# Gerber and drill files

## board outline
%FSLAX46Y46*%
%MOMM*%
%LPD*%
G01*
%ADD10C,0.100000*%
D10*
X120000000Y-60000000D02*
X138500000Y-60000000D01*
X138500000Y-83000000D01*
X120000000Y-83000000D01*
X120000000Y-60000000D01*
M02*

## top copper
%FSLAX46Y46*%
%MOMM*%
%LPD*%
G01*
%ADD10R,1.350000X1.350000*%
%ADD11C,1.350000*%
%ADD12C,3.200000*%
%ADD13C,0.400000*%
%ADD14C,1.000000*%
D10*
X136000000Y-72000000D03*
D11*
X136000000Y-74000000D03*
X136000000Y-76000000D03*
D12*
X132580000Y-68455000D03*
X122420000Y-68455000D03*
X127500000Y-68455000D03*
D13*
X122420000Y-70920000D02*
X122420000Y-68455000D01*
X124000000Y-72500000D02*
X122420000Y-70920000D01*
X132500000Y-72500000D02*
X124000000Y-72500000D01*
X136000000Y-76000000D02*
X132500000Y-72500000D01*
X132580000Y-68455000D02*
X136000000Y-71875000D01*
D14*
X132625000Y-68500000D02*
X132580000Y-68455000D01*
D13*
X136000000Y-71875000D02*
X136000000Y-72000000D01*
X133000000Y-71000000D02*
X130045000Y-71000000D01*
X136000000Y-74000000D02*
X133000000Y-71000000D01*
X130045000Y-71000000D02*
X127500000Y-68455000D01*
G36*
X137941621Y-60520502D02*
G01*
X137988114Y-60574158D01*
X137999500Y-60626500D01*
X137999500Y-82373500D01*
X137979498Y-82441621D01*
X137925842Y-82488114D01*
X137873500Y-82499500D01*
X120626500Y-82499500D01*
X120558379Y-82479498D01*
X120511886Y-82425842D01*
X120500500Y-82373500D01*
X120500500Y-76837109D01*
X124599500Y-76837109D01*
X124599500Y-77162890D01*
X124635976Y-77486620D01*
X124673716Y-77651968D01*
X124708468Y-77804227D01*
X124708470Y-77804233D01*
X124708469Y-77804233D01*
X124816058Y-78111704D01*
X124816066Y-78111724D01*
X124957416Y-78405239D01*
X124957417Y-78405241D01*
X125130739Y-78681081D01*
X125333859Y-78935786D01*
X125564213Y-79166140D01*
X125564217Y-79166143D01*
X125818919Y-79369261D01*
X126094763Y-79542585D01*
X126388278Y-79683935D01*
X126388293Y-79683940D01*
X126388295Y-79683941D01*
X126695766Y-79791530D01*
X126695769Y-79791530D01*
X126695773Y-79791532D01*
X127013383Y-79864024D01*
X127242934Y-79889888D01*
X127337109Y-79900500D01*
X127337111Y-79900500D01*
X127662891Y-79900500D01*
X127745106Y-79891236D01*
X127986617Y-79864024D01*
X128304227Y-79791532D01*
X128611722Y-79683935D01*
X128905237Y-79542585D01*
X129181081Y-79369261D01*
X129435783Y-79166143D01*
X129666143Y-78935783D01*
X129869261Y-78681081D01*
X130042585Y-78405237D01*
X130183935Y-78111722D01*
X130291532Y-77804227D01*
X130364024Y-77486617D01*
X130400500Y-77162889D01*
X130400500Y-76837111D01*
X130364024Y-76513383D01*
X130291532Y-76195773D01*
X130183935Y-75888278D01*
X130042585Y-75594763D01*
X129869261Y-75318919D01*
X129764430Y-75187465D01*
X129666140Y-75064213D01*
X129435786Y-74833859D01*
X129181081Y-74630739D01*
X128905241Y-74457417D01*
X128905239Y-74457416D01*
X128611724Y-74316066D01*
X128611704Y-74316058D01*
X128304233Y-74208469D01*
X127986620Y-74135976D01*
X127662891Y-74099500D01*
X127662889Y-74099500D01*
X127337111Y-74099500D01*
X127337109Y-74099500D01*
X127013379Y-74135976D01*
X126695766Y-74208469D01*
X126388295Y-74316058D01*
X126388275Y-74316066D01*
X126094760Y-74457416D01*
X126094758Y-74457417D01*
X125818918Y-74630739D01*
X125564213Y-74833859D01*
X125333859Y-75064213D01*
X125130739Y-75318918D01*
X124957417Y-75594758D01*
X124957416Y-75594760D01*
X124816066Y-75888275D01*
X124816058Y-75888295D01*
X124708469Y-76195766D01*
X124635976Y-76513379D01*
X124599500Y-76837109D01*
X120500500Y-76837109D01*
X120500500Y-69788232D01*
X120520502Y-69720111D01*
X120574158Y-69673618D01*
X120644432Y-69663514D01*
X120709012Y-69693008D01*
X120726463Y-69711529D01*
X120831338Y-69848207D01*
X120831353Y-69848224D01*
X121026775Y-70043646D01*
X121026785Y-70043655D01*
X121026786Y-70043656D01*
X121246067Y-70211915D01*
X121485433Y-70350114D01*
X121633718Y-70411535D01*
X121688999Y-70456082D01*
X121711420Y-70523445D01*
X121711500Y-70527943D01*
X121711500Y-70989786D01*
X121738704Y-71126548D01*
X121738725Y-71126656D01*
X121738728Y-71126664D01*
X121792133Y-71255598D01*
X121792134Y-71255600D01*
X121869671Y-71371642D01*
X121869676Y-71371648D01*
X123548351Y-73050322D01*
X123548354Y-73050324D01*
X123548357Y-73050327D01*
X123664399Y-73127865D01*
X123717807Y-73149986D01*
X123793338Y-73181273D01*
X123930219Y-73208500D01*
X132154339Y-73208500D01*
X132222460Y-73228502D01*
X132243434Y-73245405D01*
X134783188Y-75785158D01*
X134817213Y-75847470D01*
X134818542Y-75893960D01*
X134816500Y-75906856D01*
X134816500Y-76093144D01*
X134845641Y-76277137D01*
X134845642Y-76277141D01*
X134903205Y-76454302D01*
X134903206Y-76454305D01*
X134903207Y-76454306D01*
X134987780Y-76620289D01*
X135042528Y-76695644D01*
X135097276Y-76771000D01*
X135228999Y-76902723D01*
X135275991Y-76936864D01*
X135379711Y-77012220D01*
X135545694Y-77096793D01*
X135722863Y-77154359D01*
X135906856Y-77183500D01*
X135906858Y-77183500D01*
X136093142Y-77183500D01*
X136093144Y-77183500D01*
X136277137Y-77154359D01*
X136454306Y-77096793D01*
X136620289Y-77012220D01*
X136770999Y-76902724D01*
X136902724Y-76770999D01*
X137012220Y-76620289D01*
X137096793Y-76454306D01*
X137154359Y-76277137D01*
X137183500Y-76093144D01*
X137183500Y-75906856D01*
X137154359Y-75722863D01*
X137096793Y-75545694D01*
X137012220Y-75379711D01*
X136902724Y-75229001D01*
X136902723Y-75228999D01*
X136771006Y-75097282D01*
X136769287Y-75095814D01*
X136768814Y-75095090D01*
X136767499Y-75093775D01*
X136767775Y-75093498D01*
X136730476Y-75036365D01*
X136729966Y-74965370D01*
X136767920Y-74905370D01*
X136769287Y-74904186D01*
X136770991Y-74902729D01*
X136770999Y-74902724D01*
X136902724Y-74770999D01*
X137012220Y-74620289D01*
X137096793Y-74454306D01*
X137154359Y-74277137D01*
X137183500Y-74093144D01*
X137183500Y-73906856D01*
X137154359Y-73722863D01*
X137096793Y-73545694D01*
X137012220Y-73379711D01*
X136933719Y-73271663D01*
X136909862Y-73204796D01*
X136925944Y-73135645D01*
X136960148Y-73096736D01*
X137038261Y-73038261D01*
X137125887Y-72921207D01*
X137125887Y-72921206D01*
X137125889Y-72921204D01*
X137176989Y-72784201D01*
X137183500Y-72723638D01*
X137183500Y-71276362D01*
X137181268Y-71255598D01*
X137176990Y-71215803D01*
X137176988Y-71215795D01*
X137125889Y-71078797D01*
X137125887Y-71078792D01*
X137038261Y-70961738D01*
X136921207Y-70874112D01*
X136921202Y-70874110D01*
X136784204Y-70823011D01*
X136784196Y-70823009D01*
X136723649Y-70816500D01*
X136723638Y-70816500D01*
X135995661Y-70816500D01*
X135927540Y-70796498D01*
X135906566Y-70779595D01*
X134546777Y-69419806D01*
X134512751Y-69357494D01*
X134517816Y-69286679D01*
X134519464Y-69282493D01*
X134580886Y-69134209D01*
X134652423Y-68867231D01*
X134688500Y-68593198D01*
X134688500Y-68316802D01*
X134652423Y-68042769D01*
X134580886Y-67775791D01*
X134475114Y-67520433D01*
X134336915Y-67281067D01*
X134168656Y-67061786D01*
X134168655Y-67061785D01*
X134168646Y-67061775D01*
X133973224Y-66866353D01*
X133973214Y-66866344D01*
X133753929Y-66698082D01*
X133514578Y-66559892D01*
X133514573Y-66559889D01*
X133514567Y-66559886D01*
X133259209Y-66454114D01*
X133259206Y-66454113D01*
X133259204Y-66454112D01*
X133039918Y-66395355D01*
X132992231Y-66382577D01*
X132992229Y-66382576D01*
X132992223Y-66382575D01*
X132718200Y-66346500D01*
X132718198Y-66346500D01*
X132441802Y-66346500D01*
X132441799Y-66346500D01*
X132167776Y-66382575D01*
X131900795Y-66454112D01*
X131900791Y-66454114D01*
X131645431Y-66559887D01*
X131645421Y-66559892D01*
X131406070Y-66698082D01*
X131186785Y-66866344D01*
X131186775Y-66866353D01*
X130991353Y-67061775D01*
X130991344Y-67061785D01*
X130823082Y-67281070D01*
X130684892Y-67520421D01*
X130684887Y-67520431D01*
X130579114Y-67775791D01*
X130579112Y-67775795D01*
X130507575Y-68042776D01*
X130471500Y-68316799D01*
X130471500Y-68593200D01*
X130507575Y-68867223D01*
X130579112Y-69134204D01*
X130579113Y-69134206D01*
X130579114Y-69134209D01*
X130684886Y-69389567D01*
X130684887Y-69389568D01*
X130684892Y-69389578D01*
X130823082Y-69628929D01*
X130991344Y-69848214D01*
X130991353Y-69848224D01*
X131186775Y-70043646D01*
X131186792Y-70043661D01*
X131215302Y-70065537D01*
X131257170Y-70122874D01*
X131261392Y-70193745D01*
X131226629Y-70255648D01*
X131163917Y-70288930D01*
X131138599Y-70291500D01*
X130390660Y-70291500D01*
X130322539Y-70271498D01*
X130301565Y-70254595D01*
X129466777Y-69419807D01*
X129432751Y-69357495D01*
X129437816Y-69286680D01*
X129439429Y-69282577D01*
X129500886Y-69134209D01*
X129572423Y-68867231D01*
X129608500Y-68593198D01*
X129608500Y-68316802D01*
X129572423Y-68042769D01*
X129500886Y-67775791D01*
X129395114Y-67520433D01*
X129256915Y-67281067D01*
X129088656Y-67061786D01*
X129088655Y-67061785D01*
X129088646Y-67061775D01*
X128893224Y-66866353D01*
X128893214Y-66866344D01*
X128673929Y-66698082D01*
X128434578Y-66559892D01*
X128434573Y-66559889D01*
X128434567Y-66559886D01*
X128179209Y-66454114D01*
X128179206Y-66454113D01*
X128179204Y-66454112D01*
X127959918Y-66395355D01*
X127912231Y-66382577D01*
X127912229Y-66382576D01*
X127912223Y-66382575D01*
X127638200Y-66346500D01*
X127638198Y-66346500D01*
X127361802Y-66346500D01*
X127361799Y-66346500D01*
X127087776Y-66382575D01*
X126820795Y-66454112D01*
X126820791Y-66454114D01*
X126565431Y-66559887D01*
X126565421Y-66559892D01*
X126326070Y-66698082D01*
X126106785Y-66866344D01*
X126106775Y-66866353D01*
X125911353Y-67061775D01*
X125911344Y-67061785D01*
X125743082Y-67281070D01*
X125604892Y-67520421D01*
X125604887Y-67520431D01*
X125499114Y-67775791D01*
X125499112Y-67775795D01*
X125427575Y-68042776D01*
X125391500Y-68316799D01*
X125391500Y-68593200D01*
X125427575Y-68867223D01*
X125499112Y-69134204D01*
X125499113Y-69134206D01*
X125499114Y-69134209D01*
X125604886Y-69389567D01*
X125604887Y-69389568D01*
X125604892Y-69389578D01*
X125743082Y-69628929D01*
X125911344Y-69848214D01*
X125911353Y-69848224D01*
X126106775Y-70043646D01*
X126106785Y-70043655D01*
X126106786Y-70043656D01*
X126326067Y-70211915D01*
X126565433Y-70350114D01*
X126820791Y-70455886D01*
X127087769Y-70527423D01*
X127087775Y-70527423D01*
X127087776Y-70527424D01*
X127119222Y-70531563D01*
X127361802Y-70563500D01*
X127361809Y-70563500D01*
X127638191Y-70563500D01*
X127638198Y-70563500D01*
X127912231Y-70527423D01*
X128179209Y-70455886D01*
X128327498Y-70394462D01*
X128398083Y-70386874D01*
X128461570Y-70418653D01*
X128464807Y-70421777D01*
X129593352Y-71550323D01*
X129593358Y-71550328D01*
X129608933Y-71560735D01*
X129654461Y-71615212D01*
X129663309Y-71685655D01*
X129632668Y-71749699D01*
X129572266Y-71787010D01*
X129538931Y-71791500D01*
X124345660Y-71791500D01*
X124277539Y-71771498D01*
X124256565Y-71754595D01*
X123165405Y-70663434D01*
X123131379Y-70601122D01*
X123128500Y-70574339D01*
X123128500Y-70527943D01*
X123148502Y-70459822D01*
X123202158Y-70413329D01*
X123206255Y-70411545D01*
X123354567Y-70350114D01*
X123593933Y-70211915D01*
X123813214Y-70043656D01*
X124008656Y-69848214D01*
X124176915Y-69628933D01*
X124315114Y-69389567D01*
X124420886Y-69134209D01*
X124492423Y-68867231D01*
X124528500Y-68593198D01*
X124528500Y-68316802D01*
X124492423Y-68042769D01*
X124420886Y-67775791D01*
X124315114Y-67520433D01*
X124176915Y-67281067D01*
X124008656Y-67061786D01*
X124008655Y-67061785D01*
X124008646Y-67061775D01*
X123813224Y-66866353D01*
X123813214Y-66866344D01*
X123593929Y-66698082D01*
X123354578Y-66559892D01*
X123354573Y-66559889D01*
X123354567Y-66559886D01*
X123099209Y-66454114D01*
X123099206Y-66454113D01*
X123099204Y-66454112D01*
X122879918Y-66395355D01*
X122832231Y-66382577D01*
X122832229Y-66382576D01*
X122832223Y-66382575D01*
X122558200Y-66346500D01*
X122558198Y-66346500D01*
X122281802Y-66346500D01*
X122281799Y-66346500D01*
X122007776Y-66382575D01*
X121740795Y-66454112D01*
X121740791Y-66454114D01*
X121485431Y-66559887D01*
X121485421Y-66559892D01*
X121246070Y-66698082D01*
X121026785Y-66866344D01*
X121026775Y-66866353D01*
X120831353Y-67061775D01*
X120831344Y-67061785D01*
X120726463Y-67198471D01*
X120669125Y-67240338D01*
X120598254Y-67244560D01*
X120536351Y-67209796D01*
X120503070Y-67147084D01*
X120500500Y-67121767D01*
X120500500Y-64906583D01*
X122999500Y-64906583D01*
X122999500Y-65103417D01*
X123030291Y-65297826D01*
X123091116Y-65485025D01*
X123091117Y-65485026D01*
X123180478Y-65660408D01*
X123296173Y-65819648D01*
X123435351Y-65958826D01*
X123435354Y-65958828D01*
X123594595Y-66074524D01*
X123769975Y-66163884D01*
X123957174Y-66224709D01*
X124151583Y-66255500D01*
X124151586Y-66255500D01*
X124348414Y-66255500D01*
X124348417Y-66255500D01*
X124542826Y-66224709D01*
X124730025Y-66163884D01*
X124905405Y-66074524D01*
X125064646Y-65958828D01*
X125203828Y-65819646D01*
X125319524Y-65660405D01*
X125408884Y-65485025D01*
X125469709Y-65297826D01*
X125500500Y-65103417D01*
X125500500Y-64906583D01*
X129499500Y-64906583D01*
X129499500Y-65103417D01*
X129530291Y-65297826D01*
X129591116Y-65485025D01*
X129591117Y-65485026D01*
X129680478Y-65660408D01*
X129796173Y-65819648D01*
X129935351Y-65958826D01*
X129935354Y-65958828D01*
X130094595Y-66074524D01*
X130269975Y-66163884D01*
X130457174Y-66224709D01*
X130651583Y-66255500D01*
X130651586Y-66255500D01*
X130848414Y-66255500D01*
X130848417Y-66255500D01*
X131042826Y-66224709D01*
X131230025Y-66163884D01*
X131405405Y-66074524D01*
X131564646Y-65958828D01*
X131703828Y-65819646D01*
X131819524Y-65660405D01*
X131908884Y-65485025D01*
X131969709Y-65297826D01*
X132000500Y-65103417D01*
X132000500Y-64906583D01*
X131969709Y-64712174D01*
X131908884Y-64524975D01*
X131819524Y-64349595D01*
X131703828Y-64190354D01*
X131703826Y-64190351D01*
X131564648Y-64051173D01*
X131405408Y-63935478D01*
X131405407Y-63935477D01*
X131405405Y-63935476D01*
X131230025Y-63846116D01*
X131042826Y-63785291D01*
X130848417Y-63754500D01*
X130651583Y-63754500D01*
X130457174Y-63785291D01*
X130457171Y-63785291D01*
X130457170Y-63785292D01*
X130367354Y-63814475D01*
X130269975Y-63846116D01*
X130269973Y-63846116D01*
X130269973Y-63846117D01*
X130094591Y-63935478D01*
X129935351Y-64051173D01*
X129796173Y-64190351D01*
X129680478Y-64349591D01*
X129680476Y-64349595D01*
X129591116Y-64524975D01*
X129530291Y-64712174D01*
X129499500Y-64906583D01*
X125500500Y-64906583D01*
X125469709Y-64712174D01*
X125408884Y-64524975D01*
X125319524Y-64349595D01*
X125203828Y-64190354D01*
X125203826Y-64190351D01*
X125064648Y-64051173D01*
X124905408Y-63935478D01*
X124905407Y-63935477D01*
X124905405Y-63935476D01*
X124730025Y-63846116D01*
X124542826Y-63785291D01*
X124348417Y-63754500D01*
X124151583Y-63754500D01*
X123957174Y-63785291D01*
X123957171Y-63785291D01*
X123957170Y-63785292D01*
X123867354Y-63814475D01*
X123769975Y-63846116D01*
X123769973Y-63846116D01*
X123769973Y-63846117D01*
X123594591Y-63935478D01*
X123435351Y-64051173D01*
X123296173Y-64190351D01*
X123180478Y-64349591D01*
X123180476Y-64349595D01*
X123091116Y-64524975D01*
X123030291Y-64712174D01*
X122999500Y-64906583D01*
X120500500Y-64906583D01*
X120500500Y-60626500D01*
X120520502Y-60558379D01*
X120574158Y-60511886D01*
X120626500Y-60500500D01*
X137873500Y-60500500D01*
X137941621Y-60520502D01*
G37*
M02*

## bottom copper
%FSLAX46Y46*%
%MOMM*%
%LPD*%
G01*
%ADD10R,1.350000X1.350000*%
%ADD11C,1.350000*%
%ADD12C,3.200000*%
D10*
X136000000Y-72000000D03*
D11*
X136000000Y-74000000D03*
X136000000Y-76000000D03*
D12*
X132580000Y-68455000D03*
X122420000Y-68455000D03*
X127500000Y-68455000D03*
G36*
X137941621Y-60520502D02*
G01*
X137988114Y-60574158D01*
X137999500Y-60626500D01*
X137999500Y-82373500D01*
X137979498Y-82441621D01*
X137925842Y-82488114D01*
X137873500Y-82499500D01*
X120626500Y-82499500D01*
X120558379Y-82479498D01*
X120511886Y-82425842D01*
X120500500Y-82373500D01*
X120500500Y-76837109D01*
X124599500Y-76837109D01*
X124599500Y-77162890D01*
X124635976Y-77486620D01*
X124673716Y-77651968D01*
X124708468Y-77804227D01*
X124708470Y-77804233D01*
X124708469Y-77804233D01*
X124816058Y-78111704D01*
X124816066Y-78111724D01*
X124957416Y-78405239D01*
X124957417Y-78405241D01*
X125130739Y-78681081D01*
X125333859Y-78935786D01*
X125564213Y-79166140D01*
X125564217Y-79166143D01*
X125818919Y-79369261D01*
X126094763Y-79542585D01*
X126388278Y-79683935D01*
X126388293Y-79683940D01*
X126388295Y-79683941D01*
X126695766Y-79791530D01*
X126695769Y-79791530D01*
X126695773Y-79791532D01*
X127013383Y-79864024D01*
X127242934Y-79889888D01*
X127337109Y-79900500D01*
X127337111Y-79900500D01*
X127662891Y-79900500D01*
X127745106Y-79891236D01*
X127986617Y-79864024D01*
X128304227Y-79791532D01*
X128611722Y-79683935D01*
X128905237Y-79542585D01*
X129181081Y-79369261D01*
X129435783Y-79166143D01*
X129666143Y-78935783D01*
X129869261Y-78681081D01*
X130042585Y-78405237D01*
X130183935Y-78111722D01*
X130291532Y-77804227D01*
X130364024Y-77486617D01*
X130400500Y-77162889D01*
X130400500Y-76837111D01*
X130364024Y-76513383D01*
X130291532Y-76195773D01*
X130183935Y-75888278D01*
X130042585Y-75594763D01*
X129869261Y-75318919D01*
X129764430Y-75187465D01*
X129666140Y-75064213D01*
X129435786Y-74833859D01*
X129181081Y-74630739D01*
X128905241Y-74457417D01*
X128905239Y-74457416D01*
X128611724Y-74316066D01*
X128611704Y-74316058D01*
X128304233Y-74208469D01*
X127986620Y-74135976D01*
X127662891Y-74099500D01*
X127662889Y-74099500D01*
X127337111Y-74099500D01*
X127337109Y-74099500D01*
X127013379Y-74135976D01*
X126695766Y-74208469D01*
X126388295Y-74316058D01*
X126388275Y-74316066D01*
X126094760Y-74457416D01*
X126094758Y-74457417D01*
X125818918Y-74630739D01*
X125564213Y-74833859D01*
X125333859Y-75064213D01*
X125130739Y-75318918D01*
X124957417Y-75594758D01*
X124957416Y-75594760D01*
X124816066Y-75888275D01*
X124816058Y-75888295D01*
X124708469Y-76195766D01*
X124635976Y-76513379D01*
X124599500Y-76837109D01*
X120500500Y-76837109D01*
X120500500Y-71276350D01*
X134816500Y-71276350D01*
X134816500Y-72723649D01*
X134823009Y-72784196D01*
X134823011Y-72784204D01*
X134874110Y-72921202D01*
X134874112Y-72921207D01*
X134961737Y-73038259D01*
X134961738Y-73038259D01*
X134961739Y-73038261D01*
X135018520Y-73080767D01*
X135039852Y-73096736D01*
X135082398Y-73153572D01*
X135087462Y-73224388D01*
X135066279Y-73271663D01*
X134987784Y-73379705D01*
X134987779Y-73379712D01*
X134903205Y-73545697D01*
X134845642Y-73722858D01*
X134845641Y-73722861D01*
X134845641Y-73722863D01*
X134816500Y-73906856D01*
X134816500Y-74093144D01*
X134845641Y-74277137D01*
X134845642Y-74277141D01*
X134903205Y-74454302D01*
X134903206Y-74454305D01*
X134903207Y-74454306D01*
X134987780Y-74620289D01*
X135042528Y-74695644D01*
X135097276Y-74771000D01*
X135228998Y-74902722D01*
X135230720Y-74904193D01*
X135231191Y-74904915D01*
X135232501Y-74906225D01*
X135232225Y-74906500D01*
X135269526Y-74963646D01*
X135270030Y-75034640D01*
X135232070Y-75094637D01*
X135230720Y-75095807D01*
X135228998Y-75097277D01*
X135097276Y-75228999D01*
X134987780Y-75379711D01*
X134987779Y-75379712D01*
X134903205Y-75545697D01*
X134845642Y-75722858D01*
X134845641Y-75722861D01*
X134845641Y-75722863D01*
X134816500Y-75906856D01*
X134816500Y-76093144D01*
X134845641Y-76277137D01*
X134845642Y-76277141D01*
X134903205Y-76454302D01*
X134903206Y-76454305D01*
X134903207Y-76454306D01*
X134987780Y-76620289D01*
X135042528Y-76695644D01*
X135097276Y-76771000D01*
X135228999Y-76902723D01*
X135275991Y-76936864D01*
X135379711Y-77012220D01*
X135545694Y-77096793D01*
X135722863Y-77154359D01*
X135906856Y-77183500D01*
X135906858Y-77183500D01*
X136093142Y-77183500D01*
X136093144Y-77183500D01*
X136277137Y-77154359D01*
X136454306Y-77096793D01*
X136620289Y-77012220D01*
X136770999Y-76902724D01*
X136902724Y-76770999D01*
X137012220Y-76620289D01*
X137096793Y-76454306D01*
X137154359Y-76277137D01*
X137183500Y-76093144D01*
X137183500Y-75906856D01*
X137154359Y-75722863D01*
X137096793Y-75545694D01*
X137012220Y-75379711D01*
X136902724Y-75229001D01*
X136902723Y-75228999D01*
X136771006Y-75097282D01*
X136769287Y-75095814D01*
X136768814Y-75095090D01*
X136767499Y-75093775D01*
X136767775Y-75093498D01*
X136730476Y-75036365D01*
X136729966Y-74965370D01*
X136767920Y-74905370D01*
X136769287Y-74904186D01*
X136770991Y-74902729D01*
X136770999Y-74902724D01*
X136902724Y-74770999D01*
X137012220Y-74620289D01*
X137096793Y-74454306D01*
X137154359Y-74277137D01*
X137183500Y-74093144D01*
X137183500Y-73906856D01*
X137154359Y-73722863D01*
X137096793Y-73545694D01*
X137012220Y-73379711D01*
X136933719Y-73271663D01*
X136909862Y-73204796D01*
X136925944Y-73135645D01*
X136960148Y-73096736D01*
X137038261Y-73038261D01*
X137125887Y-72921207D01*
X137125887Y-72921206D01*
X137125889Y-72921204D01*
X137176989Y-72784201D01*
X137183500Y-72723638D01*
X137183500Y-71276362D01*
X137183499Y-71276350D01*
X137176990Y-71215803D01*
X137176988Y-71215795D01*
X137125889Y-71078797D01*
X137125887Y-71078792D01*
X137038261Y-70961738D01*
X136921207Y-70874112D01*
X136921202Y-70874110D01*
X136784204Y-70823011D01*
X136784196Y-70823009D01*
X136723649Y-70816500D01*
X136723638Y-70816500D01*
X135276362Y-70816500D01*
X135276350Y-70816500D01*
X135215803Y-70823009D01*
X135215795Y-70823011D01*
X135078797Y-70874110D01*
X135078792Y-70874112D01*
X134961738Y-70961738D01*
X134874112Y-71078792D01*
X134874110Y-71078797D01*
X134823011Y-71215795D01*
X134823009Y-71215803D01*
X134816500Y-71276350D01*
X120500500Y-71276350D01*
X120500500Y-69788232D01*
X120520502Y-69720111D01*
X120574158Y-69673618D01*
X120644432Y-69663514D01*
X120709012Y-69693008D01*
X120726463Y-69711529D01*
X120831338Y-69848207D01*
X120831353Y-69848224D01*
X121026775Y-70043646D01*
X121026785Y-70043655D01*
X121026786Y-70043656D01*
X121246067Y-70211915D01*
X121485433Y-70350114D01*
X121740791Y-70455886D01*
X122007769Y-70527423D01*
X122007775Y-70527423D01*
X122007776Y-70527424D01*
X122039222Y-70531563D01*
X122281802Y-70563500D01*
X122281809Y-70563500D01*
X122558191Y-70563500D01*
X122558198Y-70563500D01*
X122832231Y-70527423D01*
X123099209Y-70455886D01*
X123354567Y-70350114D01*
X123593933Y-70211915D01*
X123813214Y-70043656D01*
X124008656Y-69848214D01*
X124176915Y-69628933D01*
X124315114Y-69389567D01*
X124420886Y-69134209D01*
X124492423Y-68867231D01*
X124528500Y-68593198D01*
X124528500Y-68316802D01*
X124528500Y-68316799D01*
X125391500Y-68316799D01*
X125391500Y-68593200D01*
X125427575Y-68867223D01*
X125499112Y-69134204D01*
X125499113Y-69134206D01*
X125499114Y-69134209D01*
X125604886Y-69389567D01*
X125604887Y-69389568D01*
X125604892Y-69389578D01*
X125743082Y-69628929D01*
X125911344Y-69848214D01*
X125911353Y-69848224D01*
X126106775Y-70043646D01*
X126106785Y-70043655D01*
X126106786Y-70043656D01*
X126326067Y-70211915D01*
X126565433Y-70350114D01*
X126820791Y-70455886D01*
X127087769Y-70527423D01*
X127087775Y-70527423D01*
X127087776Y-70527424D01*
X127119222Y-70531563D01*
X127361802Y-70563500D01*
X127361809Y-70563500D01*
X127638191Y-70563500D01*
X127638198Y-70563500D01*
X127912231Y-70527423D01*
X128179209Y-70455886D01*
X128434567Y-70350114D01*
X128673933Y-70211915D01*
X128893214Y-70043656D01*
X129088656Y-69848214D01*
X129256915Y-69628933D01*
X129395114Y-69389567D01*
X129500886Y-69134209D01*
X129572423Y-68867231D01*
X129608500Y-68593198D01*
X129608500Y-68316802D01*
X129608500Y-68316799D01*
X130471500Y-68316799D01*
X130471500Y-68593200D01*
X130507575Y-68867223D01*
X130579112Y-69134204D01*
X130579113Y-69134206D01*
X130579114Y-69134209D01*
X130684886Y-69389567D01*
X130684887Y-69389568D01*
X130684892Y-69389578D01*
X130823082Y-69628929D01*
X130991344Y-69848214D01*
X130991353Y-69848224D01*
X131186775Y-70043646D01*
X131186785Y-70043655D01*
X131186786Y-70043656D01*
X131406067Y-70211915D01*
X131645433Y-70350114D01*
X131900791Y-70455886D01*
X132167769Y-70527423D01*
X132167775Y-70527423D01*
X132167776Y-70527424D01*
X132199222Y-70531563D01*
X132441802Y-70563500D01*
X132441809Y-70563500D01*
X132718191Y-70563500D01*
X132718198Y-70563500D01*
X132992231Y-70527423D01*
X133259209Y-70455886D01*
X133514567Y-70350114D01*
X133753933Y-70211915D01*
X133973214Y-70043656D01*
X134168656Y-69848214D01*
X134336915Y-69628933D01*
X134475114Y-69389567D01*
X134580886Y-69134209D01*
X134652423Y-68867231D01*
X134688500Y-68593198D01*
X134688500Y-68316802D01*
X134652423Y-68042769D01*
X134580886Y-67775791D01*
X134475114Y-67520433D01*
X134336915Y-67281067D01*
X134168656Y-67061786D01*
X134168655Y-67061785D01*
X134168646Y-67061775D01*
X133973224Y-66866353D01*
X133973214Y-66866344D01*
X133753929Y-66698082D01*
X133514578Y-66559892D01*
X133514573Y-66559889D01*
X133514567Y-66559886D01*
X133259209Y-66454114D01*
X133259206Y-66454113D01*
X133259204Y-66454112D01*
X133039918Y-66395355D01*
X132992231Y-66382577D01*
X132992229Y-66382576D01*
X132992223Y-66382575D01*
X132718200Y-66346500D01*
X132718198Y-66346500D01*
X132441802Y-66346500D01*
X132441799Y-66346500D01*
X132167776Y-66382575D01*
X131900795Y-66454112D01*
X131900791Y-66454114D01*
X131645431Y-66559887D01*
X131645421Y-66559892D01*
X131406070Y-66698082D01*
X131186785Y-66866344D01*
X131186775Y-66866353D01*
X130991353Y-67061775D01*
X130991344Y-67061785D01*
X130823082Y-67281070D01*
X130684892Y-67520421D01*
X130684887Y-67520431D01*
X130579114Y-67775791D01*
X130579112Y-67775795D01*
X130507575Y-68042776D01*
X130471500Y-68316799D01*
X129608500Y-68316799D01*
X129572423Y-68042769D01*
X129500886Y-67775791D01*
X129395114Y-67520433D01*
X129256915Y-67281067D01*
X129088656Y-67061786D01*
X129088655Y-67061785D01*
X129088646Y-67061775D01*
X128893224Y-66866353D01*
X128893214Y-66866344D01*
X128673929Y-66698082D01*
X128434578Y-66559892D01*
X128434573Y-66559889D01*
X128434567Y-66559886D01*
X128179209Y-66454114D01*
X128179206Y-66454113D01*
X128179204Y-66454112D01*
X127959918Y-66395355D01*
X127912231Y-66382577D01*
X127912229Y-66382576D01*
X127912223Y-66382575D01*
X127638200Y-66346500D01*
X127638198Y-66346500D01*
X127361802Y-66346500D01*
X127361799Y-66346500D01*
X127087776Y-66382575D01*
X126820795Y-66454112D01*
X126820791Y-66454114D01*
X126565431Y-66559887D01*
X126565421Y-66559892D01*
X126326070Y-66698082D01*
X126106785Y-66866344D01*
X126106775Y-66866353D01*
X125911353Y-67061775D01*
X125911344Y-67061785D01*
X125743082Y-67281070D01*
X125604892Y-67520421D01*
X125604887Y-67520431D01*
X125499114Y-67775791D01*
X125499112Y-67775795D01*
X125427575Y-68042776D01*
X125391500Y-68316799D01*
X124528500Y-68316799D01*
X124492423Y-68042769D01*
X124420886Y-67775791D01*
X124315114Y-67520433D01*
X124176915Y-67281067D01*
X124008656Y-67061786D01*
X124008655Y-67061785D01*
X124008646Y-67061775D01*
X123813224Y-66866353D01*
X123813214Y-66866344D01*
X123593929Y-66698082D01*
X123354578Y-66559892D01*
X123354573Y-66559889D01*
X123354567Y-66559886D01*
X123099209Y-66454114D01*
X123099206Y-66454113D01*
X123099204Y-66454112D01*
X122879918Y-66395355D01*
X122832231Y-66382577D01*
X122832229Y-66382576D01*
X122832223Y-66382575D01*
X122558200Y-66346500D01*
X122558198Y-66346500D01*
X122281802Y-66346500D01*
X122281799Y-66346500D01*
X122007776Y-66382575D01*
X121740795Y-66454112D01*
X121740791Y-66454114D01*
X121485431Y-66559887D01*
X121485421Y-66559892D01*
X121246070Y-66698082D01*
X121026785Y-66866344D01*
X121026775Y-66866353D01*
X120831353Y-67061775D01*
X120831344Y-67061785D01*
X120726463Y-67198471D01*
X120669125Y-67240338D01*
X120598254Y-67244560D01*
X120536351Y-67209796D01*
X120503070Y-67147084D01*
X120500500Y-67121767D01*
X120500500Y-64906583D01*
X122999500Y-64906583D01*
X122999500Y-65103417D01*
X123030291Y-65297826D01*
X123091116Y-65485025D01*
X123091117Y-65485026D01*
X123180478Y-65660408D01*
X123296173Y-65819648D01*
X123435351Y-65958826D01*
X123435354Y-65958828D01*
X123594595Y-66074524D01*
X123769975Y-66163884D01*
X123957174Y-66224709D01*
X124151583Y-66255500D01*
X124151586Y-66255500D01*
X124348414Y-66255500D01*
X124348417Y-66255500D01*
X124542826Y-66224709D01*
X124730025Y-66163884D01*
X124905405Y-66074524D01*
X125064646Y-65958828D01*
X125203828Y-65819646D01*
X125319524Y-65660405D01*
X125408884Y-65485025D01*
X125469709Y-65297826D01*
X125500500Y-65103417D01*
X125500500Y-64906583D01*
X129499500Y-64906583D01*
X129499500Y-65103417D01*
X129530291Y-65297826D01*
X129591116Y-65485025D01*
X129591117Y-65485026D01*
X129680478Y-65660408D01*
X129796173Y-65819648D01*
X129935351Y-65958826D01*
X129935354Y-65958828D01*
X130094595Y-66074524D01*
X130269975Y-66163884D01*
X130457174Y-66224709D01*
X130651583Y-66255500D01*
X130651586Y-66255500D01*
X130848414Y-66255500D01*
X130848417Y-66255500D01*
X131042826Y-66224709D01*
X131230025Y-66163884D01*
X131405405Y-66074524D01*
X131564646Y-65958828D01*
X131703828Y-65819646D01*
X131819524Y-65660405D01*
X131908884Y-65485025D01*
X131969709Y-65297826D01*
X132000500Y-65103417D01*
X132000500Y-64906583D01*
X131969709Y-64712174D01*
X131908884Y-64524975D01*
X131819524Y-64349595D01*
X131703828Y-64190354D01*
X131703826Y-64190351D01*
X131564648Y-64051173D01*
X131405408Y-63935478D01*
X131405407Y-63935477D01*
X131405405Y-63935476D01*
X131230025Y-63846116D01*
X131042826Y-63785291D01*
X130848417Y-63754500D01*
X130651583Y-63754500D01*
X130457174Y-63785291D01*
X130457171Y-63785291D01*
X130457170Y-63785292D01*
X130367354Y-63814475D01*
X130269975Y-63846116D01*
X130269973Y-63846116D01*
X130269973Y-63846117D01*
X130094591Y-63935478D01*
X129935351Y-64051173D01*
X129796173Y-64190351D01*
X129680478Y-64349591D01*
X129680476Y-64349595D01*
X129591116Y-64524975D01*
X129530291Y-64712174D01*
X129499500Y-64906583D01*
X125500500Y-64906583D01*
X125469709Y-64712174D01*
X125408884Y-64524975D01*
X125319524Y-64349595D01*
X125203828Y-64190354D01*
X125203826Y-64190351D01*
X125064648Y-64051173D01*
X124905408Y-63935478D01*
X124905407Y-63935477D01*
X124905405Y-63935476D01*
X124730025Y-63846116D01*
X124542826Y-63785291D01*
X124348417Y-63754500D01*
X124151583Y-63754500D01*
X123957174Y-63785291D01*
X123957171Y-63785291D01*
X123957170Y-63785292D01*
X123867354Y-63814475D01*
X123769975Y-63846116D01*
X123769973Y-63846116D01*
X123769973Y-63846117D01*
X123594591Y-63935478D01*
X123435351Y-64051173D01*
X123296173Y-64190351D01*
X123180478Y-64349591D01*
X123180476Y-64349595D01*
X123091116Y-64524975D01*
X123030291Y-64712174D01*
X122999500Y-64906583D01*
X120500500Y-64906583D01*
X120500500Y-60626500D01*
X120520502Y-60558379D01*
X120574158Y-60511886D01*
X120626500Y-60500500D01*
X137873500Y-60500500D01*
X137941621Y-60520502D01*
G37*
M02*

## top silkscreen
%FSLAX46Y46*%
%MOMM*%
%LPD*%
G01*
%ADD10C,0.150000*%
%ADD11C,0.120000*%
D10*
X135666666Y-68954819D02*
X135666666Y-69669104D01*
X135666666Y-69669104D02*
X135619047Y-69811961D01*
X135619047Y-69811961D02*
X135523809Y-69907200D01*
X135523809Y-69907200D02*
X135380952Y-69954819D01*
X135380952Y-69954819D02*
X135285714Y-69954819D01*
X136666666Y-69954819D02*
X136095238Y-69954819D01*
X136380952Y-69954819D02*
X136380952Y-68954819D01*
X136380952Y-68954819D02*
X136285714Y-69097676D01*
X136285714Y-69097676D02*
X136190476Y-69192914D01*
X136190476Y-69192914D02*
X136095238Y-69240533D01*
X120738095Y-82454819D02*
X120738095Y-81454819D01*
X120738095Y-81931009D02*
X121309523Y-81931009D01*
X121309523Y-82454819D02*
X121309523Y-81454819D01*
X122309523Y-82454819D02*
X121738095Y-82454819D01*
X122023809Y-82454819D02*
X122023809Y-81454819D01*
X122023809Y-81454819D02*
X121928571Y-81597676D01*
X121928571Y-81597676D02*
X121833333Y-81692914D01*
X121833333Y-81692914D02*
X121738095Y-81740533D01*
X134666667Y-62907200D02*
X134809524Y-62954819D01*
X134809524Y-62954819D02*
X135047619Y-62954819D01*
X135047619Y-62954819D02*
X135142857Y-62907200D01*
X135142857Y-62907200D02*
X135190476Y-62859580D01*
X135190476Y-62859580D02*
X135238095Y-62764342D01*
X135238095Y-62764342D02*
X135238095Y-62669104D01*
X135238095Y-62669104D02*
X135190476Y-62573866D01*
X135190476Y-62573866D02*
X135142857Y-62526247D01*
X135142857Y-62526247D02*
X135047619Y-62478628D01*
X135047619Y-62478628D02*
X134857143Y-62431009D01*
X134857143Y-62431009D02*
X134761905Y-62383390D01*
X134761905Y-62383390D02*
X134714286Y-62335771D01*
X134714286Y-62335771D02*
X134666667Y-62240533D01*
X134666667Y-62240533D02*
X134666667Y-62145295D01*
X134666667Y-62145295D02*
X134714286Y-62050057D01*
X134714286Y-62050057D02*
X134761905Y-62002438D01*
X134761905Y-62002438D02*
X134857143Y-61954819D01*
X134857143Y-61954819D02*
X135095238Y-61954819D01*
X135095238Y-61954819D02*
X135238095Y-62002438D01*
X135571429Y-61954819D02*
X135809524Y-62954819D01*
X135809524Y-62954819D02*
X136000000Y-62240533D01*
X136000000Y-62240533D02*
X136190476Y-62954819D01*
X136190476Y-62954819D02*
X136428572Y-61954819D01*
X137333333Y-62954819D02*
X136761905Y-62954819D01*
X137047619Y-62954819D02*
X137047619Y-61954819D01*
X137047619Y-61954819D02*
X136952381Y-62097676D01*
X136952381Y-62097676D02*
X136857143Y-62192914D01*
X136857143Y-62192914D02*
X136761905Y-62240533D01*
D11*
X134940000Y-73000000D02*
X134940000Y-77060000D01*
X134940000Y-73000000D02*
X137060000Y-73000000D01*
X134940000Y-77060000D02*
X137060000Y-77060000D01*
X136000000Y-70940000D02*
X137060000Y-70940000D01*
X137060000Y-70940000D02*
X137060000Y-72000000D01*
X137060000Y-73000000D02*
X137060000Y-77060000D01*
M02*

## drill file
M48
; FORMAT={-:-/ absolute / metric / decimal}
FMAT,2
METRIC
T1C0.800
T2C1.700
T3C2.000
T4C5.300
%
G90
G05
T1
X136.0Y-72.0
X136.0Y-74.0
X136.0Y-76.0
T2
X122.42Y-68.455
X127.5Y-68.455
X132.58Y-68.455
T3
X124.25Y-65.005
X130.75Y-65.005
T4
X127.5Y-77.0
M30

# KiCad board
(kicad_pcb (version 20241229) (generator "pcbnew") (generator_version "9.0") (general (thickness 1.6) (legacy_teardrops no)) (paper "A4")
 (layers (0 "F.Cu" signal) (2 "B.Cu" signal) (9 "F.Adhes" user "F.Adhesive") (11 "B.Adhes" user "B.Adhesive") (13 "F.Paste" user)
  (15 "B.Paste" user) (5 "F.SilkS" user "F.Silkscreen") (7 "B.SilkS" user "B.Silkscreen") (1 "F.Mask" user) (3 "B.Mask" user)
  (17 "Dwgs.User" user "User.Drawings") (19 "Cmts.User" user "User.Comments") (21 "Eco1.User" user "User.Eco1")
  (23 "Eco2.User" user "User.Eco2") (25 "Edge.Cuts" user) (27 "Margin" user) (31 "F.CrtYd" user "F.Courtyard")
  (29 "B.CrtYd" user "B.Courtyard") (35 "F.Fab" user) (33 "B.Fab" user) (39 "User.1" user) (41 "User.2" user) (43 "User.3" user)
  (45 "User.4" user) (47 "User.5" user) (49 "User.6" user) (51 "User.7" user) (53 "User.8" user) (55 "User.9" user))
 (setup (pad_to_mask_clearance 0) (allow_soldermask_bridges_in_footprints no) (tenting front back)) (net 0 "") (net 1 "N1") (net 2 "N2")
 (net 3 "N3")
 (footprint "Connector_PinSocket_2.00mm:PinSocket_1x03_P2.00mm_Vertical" (layer "F.Cu") (at 136 72)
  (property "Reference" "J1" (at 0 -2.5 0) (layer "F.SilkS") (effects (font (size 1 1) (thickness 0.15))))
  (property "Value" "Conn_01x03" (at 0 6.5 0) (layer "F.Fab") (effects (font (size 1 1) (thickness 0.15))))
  (fp_line (start -1.06 1) (end -1.06 5.06) (stroke (width 0.12) (type solid)) (layer "F.SilkS"))
  (fp_line (start -1.06 1) (end 1.06 1) (stroke (width 0.12) (type solid)) (layer "F.SilkS"))
  (fp_line (start -1.06 5.06) (end 1.06 5.06) (stroke (width 0.12) (type solid)) (layer "F.SilkS"))
  (fp_line (start 0 -1.06) (end 1.06 -1.06) (stroke (width 0.12) (type solid)) (layer "F.SilkS"))
  (fp_line (start 1.06 -1.06) (end 1.06 0) (stroke (width 0.12) (type solid)) (layer "F.SilkS"))
  (fp_line (start 1.06 1) (end 1.06 5.06) (stroke (width 0.12) (type solid)) (layer "F.SilkS"))
  (pad "1" thru_hole rect (at 0 0) (size 1.35 1.35) (drill 0.8) (layers "*.Cu" "*.Mask") (remove_unused_layers no) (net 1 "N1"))
  (pad "2" thru_hole circle (at 0 2) (size 1.35 1.35) (drill 0.8) (layers "*.Cu" "*.Mask") (remove_unused_layers no) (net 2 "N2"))
  (pad "3" thru_hole circle (at 0 4) (size 1.35 1.35) (drill 0.8) (layers "*.Cu" "*.Mask") (remove_unused_layers no) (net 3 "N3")))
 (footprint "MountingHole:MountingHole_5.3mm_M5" (layer "F.Cu") (at 127.5 77)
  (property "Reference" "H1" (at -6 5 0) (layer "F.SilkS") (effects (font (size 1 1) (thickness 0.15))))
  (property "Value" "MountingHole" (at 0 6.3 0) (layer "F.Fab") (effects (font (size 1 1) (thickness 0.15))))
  (pad "" np_thru_hole circle (at 0 0) (size 5.3 5.3) (drill 5.3) (layers "*.Cu" "*.Mask")))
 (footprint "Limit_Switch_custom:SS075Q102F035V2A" (layer "F.Cu") (at 127.5 68.455)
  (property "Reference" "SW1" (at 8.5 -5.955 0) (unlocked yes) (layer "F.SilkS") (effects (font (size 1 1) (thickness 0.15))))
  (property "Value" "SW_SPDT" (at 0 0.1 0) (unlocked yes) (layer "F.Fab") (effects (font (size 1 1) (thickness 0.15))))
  (pad "" np_thru_hole circle (at -3.25 -3.45) (size 2 2) (drill 2) (layers "*.Cu" "*.Mask"))
  (pad "" np_thru_hole circle (at 3.25 -3.45) (size 2 2) (drill 2) (layers "*.Cu" "*.Mask"))
  (pad "1" thru_hole circle (at 5.08 0) (size 3.2 3.2) (drill 1.7) (layers "*.Cu" "*.Mask") (remove_unused_layers no) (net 1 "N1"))
  (pad "2" thru_hole circle (at -5.08 0) (size 3.2 3.2) (drill 1.7) (layers "*.Cu" "*.Mask") (remove_unused_layers no) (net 3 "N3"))
  (pad "3" thru_hole circle (at 0 0) (size 3.2 3.2) (drill 1.7) (layers "*.Cu" "*.Mask") (remove_unused_layers no) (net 2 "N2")))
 (gr_rect (start 120 60) (end 138.5 83) (stroke (width 0.1) (type solid)) (fill no) (layer "Edge.Cuts"))
 (segment (start 122.42 70.92) (end 122.42 68.455) (width 0.4) (layer "F.Cu") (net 3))
 (segment (start 124 72.5) (end 122.42 70.92) (width 0.4) (layer "F.Cu") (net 3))
 (segment (start 132.5 72.5) (end 124 72.5) (width 0.4) (layer "F.Cu") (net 3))
 (segment (start 136 76) (end 132.5 72.5) (width 0.4) (layer "F.Cu") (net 3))
 (segment (start 132.58 68.455) (end 136 71.875) (width 0.4) (layer "F.Cu") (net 1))
 (segment (start 132.625 68.5) (end 132.58 68.455) (width 1) (layer "F.Cu") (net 1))
 (segment (start 136 71.875) (end 136 72) (width 0.4) (layer "F.Cu") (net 1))
 (segment (start 133 71) (end 130.045 71) (width 0.4) (layer "F.Cu") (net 2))
 (segment (start 136 74) (end 133 71) (width 0.4) (layer "F.Cu") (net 2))
 (segment (start 130.045 71) (end 127.5 68.455) (width 0.4) (layer "F.Cu") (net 2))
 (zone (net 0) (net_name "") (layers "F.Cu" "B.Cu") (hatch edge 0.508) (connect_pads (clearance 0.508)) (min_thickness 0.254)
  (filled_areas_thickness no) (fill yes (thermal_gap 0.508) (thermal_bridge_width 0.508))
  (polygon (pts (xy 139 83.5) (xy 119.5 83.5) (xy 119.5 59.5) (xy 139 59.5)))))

